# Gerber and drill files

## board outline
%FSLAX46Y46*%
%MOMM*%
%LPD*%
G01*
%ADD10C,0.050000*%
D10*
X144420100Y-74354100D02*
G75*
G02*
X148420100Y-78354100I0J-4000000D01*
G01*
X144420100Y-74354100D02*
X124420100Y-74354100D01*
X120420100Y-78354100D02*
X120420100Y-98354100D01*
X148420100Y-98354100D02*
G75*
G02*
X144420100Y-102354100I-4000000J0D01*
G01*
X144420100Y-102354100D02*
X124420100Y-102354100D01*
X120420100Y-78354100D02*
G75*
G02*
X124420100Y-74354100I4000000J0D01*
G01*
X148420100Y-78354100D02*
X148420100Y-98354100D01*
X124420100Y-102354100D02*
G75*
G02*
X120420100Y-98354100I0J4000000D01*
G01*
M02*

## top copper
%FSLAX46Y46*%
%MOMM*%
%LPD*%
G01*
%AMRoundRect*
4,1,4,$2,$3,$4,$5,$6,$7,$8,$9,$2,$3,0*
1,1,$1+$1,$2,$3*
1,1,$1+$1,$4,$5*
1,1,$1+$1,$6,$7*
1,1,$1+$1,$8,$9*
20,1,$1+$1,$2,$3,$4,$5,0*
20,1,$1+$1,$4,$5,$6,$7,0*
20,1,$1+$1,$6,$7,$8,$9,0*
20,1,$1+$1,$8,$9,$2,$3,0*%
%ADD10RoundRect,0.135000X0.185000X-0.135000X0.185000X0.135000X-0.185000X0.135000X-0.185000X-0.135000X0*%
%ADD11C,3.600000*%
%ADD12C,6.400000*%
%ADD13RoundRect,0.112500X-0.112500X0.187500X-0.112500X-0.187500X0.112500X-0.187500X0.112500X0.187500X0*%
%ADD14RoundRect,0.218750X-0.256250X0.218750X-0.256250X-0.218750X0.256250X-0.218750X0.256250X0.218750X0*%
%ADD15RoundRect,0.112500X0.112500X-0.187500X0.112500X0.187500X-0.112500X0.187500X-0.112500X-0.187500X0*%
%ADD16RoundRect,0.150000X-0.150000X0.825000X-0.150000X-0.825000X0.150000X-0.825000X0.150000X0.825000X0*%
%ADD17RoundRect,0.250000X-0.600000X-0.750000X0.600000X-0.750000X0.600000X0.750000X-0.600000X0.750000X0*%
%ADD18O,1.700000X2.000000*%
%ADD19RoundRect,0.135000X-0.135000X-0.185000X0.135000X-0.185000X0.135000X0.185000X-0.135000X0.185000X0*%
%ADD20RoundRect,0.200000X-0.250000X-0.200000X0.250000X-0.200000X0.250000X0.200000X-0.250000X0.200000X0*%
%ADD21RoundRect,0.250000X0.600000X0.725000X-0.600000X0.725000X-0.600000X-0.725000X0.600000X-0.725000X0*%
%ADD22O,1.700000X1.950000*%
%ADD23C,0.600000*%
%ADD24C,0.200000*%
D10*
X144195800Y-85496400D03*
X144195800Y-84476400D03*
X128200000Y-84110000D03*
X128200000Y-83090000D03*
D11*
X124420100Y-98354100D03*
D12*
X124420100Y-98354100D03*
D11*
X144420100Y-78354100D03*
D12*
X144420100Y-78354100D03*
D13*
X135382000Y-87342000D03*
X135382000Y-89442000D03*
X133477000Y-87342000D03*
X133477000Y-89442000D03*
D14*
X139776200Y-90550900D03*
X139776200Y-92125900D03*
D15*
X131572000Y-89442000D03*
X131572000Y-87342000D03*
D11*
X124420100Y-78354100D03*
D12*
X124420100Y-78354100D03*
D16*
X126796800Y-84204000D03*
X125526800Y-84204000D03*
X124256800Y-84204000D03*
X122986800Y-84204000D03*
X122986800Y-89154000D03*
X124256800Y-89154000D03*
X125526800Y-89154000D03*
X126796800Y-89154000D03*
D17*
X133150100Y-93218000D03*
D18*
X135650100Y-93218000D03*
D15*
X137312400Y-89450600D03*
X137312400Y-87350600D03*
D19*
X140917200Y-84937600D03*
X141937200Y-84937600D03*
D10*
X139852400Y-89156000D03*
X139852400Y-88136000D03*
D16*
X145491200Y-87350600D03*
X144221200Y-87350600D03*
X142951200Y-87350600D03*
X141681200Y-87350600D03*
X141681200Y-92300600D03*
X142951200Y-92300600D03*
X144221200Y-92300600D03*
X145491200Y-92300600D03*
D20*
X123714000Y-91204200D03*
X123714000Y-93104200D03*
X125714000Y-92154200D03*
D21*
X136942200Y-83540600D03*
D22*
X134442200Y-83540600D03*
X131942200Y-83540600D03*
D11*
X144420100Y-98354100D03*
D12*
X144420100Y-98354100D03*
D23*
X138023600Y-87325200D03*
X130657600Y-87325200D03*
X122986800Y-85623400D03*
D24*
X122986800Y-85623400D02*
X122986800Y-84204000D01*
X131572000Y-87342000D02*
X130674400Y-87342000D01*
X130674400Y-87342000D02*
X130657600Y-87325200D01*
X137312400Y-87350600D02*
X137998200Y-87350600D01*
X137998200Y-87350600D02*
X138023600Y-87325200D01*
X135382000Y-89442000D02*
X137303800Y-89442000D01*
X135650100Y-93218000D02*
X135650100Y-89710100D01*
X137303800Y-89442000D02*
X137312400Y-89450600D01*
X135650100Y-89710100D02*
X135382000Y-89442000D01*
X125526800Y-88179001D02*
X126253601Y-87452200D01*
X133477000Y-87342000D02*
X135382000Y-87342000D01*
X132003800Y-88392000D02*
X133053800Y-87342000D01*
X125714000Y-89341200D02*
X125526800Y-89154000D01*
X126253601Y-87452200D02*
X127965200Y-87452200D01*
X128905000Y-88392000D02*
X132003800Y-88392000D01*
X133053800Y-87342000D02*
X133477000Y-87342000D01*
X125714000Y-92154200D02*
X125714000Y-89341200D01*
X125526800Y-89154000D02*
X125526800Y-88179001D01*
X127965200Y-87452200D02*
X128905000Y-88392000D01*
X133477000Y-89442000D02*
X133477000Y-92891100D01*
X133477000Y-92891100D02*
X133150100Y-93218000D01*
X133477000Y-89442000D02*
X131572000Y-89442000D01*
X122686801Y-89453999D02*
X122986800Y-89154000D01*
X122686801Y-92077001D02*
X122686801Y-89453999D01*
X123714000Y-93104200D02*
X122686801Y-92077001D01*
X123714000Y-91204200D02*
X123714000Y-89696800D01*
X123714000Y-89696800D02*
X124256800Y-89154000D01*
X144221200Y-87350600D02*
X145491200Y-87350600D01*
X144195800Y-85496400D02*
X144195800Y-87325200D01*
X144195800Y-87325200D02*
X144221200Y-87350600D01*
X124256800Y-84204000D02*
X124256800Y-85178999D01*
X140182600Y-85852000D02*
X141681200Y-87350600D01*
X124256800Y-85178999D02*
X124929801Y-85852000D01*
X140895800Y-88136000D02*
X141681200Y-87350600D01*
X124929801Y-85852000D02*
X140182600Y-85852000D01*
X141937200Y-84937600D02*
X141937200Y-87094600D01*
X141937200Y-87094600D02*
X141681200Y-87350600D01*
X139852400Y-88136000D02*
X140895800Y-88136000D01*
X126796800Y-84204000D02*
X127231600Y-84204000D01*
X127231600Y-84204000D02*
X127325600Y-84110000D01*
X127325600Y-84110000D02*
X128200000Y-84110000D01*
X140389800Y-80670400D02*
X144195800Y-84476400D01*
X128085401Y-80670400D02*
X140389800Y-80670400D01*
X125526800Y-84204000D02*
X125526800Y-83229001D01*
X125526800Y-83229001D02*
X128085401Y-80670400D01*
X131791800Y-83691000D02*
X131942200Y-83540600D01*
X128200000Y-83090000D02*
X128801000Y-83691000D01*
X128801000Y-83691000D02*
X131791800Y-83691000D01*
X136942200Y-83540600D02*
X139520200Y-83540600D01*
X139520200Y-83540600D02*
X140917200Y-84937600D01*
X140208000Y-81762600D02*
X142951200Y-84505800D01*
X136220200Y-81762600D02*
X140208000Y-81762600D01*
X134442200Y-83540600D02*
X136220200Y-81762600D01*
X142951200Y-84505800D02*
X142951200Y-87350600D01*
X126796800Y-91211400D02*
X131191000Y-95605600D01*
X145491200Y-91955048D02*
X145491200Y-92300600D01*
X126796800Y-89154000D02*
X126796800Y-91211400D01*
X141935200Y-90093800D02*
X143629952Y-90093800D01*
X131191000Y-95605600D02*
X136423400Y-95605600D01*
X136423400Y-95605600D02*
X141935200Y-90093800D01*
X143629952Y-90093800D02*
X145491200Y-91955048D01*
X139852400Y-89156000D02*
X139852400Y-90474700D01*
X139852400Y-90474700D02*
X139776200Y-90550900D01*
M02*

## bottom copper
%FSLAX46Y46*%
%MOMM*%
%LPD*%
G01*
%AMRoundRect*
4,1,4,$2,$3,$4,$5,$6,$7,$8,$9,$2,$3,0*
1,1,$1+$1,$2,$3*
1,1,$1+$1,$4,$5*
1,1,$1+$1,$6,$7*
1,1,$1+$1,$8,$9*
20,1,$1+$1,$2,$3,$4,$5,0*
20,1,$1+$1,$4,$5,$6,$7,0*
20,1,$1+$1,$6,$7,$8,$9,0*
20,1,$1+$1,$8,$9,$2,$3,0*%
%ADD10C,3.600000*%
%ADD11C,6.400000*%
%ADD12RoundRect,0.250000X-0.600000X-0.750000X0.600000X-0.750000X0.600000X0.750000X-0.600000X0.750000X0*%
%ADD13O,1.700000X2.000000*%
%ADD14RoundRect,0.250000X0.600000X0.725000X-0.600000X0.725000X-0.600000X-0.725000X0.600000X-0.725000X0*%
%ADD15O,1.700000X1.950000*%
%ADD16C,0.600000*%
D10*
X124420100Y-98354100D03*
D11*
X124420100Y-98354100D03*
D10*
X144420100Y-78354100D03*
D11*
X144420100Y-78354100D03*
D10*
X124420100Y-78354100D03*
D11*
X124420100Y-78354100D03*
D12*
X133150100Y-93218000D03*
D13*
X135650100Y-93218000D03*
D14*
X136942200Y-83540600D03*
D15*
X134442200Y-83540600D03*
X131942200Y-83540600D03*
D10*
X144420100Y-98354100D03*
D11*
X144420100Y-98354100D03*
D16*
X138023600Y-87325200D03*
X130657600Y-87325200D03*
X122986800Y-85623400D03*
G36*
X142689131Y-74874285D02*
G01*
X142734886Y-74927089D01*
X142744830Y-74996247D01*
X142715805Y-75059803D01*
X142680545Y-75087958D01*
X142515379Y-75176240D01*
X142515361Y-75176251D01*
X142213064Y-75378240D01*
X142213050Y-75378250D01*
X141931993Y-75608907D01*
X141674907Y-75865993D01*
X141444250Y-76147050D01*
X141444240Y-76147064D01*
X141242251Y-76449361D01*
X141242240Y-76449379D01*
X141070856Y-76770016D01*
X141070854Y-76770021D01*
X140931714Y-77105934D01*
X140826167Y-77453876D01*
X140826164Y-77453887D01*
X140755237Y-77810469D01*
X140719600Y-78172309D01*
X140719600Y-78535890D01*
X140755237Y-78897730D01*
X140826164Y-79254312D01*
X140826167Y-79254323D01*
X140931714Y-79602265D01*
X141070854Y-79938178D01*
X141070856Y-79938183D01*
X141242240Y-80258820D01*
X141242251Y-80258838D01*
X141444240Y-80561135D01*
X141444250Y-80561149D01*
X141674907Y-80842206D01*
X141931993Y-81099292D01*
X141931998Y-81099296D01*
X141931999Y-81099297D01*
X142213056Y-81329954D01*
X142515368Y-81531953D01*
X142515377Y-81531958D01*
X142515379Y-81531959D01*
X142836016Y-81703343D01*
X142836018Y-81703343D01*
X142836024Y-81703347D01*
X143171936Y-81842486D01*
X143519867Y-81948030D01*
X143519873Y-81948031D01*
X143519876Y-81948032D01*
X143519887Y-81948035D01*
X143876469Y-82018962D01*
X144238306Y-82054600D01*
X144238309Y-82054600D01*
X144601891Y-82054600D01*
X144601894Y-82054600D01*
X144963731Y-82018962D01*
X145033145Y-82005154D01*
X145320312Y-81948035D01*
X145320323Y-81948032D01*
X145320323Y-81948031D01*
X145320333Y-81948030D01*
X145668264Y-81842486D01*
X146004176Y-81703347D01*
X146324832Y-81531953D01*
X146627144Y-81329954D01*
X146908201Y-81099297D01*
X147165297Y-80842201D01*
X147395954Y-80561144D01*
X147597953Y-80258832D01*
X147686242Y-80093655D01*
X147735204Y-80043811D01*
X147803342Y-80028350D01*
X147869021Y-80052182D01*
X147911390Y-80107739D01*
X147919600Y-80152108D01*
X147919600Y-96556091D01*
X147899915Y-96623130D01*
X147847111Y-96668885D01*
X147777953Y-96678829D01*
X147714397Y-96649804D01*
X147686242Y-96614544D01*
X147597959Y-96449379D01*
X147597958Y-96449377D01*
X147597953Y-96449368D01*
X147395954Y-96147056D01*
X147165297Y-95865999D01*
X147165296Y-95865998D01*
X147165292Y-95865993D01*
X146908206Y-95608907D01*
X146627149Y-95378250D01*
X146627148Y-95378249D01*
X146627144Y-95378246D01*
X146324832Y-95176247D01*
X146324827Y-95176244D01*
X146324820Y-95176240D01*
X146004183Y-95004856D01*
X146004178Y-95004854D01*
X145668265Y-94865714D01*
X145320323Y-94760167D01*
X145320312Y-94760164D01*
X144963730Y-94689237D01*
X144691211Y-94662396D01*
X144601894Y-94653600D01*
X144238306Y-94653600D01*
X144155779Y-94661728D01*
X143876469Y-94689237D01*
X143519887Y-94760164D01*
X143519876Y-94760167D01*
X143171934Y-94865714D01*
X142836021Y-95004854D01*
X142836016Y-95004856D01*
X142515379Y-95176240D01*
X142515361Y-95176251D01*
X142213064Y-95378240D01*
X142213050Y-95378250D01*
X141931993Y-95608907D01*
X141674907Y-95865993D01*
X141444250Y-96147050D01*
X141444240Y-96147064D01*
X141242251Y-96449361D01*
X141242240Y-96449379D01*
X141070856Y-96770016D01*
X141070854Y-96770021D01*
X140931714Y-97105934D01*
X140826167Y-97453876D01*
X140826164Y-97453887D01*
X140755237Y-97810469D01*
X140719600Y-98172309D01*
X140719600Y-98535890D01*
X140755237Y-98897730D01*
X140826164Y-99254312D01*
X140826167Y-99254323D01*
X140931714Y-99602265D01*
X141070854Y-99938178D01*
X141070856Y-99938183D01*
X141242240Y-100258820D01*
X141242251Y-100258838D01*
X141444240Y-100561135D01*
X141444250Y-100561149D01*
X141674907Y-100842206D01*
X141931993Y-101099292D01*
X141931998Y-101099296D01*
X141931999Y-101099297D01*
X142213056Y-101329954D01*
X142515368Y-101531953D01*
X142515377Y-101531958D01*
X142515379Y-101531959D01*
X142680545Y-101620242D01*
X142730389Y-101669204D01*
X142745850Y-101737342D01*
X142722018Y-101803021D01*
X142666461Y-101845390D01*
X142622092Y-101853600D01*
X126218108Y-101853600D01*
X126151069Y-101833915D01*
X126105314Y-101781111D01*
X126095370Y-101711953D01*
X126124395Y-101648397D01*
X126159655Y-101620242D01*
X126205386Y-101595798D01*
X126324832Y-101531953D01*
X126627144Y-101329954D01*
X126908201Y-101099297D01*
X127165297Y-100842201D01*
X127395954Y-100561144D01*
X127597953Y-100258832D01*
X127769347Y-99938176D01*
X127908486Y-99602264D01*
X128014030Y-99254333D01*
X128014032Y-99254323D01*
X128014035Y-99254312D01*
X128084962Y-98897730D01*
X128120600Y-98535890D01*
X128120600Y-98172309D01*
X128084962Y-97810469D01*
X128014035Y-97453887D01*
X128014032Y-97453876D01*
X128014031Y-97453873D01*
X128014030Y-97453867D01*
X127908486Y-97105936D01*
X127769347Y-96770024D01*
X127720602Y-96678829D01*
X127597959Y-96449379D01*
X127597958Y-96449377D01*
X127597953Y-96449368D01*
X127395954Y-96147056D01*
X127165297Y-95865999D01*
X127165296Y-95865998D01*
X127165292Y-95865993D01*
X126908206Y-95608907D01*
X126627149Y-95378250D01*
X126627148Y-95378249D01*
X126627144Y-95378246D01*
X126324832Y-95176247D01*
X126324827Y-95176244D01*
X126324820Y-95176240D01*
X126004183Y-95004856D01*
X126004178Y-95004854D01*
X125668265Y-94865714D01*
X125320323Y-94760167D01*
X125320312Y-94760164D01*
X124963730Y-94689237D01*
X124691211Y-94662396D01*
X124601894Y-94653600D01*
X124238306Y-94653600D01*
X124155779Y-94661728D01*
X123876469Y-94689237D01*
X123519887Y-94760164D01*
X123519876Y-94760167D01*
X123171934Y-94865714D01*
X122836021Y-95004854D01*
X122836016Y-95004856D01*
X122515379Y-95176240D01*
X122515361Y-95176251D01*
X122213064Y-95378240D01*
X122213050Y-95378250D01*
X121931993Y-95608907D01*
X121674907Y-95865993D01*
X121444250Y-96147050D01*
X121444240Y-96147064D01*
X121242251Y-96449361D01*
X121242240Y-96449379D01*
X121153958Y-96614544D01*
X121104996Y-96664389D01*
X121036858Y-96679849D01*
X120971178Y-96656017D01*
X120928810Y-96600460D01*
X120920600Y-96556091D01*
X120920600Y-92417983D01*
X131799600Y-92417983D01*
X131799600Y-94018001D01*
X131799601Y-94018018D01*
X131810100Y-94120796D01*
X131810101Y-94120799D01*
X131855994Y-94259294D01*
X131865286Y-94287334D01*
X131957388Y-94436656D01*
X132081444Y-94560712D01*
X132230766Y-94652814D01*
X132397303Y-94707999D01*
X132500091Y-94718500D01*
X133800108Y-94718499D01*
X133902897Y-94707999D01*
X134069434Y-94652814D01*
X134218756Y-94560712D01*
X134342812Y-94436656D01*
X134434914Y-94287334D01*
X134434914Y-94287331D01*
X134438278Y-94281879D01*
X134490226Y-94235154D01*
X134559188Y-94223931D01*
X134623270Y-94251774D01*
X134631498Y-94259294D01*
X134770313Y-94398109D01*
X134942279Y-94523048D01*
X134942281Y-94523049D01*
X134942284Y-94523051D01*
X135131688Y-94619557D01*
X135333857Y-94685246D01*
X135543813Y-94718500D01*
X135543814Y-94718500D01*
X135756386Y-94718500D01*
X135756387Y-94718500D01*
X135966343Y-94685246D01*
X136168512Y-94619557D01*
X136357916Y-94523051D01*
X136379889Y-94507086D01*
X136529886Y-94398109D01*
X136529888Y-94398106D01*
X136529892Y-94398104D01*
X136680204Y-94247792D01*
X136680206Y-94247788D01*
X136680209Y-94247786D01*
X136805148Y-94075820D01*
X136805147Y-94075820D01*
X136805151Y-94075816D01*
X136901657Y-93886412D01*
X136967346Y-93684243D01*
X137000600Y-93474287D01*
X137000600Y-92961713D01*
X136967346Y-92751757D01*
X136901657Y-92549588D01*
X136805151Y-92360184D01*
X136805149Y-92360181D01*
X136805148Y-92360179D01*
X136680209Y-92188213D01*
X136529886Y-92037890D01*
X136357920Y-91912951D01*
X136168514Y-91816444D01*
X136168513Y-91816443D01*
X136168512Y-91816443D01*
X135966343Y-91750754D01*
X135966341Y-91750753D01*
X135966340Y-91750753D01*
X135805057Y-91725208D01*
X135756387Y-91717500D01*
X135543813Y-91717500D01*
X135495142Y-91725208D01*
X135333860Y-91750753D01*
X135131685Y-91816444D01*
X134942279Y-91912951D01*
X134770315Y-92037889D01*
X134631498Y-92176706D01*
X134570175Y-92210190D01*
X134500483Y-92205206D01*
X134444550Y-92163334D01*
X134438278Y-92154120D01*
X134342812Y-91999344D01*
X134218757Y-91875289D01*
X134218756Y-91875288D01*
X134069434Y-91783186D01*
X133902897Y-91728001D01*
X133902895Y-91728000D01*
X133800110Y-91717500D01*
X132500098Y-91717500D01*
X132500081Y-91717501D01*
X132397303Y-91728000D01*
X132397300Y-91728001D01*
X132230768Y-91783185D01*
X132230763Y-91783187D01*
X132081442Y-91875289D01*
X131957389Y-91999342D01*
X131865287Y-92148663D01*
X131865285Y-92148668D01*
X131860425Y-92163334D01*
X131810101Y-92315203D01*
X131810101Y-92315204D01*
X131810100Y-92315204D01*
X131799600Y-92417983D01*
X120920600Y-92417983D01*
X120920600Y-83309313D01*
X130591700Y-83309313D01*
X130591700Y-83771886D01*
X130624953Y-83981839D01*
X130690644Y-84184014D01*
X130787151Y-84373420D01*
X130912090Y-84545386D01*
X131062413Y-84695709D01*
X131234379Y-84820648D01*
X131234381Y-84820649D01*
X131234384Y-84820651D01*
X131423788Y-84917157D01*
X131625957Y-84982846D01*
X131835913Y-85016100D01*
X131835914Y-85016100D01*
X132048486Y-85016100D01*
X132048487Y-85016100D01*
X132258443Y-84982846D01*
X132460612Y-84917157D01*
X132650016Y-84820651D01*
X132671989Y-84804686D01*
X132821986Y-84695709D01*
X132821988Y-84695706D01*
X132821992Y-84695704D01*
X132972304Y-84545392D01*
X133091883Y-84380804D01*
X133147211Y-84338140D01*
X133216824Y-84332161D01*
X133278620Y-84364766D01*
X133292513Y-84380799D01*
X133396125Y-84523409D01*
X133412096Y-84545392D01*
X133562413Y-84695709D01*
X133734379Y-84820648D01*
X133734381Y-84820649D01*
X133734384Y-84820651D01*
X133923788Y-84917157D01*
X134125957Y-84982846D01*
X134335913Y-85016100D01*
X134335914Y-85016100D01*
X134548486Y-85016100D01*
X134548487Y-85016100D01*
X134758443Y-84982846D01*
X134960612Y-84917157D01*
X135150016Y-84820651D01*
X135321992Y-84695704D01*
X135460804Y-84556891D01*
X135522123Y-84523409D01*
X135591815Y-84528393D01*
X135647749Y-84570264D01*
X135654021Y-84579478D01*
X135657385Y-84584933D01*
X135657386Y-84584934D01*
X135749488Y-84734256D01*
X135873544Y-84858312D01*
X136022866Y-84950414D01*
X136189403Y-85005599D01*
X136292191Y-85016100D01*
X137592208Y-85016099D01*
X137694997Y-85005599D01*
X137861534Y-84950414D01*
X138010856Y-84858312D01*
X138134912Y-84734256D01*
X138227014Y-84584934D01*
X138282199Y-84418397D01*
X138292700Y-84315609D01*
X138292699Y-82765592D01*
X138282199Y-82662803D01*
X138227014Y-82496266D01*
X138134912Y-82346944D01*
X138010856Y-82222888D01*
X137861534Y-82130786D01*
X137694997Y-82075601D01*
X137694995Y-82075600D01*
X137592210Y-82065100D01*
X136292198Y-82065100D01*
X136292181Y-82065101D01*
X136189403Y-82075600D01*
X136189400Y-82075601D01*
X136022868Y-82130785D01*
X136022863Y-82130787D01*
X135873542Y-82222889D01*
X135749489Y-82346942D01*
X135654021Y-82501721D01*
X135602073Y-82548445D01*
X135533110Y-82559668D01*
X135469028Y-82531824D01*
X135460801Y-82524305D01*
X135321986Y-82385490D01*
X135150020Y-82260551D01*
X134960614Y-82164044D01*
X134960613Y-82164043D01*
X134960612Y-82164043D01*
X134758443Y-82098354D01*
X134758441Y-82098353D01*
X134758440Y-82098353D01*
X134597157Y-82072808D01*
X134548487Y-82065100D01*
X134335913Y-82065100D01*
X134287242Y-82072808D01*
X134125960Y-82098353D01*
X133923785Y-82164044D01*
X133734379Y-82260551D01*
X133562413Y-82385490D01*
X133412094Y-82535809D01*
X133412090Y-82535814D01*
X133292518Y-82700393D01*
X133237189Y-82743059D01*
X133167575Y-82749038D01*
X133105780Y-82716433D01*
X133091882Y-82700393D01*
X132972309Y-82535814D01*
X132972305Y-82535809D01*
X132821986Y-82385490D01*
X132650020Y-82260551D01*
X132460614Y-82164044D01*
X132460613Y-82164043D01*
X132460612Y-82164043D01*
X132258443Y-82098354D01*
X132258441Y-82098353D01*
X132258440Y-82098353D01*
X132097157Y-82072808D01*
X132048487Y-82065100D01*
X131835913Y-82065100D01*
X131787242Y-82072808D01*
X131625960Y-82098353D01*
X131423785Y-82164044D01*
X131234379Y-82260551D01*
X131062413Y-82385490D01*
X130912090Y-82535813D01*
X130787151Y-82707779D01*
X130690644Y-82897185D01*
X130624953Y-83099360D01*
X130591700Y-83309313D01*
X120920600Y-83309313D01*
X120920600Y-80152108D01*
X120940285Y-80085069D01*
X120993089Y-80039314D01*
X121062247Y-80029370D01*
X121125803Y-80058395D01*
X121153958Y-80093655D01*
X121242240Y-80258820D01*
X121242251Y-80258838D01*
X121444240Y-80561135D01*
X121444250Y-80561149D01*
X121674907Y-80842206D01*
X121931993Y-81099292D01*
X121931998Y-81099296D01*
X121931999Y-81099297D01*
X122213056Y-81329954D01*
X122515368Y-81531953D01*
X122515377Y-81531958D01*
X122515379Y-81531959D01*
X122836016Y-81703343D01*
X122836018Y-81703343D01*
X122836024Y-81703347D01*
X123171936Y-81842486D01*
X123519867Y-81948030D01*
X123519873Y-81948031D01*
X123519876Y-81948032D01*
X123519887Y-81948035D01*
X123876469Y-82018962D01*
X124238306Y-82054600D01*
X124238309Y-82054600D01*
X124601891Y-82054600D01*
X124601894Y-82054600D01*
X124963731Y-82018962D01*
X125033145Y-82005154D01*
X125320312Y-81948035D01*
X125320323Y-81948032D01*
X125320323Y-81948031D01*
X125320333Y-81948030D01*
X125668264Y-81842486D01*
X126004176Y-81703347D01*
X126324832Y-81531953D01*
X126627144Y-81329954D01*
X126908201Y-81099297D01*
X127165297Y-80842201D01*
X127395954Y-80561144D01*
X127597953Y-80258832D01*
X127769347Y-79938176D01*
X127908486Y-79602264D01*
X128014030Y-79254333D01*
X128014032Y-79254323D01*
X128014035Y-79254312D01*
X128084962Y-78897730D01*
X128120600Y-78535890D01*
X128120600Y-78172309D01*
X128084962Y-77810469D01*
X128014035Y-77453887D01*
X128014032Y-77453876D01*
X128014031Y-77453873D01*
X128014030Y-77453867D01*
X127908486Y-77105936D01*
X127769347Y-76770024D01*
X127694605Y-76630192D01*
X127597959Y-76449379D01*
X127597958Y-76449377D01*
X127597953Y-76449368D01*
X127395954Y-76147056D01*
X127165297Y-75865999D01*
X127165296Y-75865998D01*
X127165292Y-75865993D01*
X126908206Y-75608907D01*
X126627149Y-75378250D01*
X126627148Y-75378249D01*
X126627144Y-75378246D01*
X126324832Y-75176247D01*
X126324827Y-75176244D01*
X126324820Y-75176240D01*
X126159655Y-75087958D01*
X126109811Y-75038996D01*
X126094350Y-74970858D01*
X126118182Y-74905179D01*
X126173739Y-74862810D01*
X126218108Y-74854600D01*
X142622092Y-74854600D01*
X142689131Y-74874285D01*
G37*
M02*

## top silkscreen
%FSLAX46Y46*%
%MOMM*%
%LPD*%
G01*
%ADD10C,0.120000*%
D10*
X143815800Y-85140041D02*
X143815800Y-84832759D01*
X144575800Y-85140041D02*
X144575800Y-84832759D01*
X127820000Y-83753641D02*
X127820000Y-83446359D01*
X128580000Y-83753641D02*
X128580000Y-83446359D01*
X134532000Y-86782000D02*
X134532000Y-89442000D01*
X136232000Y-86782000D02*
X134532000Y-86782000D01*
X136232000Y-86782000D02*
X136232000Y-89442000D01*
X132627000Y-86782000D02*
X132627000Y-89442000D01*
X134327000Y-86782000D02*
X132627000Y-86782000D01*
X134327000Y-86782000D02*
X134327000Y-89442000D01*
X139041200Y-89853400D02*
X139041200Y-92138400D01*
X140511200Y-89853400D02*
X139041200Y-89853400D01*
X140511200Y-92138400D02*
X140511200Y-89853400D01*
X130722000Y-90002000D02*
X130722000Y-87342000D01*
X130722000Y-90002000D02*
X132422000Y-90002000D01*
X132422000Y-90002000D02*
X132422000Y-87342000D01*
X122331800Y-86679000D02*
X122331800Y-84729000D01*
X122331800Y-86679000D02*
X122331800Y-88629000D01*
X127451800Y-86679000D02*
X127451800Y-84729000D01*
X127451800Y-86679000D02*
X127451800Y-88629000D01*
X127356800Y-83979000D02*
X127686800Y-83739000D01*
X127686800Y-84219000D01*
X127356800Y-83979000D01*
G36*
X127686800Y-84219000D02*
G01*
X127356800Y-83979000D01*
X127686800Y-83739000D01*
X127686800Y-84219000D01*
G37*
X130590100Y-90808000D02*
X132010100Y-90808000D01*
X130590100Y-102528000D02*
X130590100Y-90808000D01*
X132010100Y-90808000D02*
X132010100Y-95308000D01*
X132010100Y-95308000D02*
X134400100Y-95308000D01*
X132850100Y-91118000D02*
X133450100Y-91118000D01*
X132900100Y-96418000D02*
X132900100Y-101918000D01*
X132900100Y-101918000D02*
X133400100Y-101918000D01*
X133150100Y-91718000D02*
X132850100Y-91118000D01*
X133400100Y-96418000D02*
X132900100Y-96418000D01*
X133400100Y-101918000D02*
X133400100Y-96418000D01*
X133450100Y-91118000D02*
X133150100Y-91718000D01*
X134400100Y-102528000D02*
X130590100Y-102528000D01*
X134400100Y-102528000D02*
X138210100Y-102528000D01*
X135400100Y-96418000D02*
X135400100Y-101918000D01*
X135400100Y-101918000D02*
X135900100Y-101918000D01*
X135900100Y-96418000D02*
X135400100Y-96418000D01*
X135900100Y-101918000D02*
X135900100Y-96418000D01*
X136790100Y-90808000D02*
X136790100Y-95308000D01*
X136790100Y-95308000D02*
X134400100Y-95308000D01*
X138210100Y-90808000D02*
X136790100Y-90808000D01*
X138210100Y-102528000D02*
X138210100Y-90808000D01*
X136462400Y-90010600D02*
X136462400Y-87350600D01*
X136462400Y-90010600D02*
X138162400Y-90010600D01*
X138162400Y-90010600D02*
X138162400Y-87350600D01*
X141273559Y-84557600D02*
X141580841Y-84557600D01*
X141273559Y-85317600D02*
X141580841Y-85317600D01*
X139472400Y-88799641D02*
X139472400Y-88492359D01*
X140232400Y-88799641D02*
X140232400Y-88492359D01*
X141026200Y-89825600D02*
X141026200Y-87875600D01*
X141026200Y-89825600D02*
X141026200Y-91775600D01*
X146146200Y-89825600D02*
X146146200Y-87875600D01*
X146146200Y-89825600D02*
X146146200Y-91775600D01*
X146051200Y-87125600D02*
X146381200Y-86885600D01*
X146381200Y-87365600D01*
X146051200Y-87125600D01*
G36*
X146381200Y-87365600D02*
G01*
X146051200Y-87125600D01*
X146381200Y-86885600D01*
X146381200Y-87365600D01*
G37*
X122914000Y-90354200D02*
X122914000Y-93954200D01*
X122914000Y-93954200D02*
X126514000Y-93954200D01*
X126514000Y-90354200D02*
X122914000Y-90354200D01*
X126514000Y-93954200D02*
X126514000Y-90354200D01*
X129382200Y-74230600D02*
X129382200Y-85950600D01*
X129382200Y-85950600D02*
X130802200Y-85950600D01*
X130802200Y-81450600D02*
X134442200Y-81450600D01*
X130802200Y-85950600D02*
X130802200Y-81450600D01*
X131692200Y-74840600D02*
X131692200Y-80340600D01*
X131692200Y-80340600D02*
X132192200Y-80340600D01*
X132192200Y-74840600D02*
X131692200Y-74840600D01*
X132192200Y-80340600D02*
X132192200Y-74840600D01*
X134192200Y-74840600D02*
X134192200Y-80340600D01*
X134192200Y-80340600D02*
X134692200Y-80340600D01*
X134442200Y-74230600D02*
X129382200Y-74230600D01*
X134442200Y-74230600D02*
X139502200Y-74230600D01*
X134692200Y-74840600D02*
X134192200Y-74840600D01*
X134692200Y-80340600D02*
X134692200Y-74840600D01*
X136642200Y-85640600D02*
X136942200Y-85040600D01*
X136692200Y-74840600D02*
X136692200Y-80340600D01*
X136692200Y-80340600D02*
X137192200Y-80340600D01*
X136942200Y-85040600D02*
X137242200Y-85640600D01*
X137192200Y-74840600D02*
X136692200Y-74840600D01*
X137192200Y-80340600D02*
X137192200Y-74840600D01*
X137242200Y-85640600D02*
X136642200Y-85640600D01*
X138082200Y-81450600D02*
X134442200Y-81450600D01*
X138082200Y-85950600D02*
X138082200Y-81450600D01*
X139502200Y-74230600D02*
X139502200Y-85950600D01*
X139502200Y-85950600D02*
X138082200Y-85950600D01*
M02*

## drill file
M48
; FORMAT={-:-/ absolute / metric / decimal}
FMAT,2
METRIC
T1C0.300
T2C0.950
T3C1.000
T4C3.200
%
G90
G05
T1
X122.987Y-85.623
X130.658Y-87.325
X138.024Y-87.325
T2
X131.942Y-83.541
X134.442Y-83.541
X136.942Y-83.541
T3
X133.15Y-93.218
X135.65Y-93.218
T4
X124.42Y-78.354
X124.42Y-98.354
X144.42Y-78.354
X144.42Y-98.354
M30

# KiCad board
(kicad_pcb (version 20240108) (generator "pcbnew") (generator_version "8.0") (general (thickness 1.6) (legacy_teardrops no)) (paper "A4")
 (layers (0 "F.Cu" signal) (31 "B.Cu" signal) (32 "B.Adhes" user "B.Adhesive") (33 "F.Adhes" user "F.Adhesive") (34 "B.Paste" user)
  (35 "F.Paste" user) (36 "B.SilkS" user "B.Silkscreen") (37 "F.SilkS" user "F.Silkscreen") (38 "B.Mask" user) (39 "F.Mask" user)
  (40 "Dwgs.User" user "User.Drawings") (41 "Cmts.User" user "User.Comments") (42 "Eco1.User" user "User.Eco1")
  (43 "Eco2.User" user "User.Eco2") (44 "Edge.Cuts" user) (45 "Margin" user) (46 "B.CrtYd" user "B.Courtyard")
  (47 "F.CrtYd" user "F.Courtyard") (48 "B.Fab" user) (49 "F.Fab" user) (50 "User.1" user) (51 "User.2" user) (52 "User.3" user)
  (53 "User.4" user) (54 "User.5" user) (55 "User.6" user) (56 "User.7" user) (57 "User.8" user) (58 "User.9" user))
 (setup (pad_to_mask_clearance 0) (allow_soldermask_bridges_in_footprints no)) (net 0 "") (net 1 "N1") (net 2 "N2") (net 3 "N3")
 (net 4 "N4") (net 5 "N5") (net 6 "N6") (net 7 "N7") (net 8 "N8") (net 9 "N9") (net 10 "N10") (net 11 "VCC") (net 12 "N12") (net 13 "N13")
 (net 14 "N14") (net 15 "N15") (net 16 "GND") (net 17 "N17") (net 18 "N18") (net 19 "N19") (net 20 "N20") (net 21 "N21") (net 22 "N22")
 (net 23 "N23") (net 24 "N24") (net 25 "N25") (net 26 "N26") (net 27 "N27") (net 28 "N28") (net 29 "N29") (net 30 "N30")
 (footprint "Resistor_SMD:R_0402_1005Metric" (layer "F.Cu") (at 144.1958 84.9864 90)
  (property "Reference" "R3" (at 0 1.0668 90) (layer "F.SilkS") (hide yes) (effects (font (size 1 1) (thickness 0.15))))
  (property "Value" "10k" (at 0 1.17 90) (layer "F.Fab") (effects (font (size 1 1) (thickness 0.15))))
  (fp_line (start -0.153641 -0.38) (end 0.153641 -0.38) (stroke (width 0.12) (type solid)) (layer "F.SilkS"))
  (fp_line (start -0.153641 0.38) (end 0.153641 0.38) (stroke (width 0.12) (type solid)) (layer "F.SilkS"))
  (pad "1" smd roundrect (at -0.51 0 90) (size 0.54 0.64) (layers "F.Cu" "F.Paste" "F.Mask") (roundrect_rratio 0.25) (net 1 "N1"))
  (pad "2" smd roundrect (at 0.51 0 90) (size 0.54 0.64) (layers "F.Cu" "F.Paste" "F.Mask") (roundrect_rratio 0.25) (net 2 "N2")))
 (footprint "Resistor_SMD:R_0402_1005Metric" (layer "F.Cu") (at 128.2 83.6 90)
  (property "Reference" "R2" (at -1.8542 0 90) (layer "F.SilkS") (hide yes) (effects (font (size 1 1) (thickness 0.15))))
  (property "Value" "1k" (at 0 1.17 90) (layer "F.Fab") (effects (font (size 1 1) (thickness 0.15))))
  (fp_line (start -0.153641 -0.38) (end 0.153641 -0.38) (stroke (width 0.12) (type solid)) (layer "F.SilkS"))
  (fp_line (start -0.153641 0.38) (end 0.153641 0.38) (stroke (width 0.12) (type solid)) (layer "F.SilkS"))
  (pad "1" smd roundrect (at -0.51 0 90) (size 0.54 0.64) (layers "F.Cu" "F.Paste" "F.Mask") (roundrect_rratio 0.25) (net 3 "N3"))
  (pad "2" smd roundrect (at 0.51 0 90) (size 0.54 0.64) (layers "F.Cu" "F.Paste" "F.Mask") (roundrect_rratio 0.25) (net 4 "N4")))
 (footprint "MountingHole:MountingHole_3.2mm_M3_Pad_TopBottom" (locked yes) (layer "F.Cu") (at 124.4201 98.3541)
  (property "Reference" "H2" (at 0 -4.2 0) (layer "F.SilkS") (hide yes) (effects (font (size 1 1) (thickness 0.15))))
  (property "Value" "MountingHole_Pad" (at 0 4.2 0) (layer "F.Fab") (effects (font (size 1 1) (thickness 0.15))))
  (pad "1" thru_hole circle (at 0 0) (size 3.6 3.6) (drill 3.2) (layers "*.Cu" "*.Mask") (remove_unused_layers no) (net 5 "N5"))
  (pad "1" connect circle (at 0 0) (size 6.4 6.4) (layers "F.Cu" "F.Mask") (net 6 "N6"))
  (pad "1" connect circle (at 0 0) (size 6.4 6.4) (layers "B.Cu" "B.Mask") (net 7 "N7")))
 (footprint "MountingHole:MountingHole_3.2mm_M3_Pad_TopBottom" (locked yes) (layer "F.Cu") (at 144.4201 78.3541)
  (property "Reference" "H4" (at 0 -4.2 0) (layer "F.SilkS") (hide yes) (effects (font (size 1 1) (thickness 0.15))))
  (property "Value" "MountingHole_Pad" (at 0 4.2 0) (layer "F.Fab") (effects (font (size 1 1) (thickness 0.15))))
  (pad "1" thru_hole circle (at 0 0) (size 3.6 3.6) (drill 3.2) (layers "*.Cu" "*.Mask") (remove_unused_layers no) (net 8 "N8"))
  (pad "1" connect circle (at 0 0) (size 6.4 6.4) (layers "F.Cu" "F.Mask") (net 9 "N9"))
  (pad "1" connect circle (at 0 0) (size 6.4 6.4) (layers "B.Cu" "B.Mask") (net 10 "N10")))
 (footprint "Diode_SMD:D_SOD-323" (layer "F.Cu") (at 135.382 88.392 -90)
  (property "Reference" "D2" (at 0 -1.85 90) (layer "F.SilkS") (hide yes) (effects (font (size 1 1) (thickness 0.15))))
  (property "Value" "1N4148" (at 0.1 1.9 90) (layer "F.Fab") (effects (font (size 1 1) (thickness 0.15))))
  (fp_line (start -1.61 0.85) (end 1.05 0.85) (stroke (width 0.12) (type solid)) (layer "F.SilkS"))
  (fp_line (start -1.61 -0.85) (end -1.61 0.85) (stroke (width 0.12) (type solid)) (layer "F.SilkS"))
  (fp_line (start -1.61 -0.85) (end 1.05 -0.85) (stroke (width 0.12) (type solid)) (layer "F.SilkS"))
  (pad "1" smd roundrect (at -1.05 0 270) (size 0.6 0.45) (layers "F.Cu" "F.Paste" "F.Mask") (roundrect_rratio 0.25) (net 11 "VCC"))
  (pad "2" smd roundrect (at 1.05 0 270) (size 0.6 0.45) (layers "F.Cu" "F.Paste" "F.Mask") (roundrect_rratio 0.25) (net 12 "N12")))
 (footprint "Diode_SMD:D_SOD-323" (layer "F.Cu") (at 133.477 88.392 -90)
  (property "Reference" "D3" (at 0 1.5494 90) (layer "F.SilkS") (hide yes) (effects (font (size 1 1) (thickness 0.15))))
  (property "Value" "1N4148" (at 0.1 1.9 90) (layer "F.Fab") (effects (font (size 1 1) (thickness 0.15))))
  (fp_line (start -1.61 0.85) (end 1.05 0.85) (stroke (width 0.12) (type solid)) (layer "F.SilkS"))
  (fp_line (start -1.61 -0.85) (end -1.61 0.85) (stroke (width 0.12) (type solid)) (layer "F.SilkS"))
  (fp_line (start -1.61 -0.85) (end 1.05 -0.85) (stroke (width 0.12) (type solid)) (layer "F.SilkS"))
  (pad "1" smd roundrect (at -1.05 0 270) (size 0.6 0.45) (layers "F.Cu" "F.Paste" "F.Mask") (roundrect_rratio 0.25) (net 11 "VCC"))
  (pad "2" smd roundrect (at 1.05 0 270) (size 0.6 0.45) (layers "F.Cu" "F.Paste" "F.Mask") (roundrect_rratio 0.25) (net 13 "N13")))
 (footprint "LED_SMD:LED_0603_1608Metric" (layer "F.Cu") (at 139.7762 91.3384 -90)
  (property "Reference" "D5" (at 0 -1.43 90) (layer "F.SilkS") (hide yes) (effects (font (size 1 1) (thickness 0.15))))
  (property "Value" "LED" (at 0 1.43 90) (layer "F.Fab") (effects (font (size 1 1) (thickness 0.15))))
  (fp_line (start -1.485 0.735) (end 0.8 0.735) (stroke (width 0.12) (type solid)) (layer "F.SilkS"))
  (fp_line (start -1.485 -0.735) (end -1.485 0.735) (stroke (width 0.12) (type solid)) (layer "F.SilkS"))
  (fp_line (start 0.8 -0.735) (end -1.485 -0.735) (stroke (width 0.12) (type solid)) (layer "F.SilkS"))
  (pad "1" smd roundrect (at -0.7875 0 270) (size 0.875 0.95) (layers "F.Cu" "F.Paste" "F.Mask") (roundrect_rratio 0.25) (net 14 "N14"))
  (pad "2" smd roundrect (at 0.7875 0 270) (size 0.875 0.95) (layers "F.Cu" "F.Paste" "F.Mask") (roundrect_rratio 0.25) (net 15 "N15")))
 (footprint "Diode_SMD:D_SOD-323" (layer "F.Cu") (at 131.572 88.392 90)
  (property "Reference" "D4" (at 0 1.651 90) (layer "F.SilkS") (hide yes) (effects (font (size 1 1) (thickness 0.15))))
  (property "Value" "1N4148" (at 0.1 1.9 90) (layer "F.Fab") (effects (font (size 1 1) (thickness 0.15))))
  (fp_line (start -1.61 -0.85) (end 1.05 -0.85) (stroke (width 0.12) (type solid)) (layer "F.SilkS"))
  (fp_line (start -1.61 -0.85) (end -1.61 0.85) (stroke (width 0.12) (type solid)) (layer "F.SilkS"))
  (fp_line (start -1.61 0.85) (end 1.05 0.85) (stroke (width 0.12) (type solid)) (layer "F.SilkS"))
  (pad "1" smd roundrect (at -1.05 0 90) (size 0.6 0.45) (layers "F.Cu" "F.Paste" "F.Mask") (roundrect_rratio 0.25) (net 13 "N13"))
  (pad "2" smd roundrect (at 1.05 0 90) (size 0.6 0.45) (layers "F.Cu" "F.Paste" "F.Mask") (roundrect_rratio 0.25) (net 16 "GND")))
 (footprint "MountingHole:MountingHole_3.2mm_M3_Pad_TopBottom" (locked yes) (layer "F.Cu") (at 124.4201 78.3541)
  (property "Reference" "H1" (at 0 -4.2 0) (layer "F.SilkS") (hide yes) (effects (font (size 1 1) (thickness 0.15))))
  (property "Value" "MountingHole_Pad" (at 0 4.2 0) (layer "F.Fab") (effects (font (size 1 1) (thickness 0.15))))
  (pad "1" thru_hole circle (at 0 0) (size 3.6 3.6) (drill 3.2) (layers "*.Cu" "*.Mask") (remove_unused_layers no) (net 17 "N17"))
  (pad "1" connect circle (at 0 0) (size 6.4 6.4) (layers "F.Cu" "F.Mask") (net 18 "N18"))
  (pad "1" connect circle (at 0 0) (size 6.4 6.4) (layers "B.Cu" "B.Mask") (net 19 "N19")))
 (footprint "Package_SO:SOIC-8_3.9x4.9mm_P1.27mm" (layer "F.Cu") (at 124.8918 86.679 -90)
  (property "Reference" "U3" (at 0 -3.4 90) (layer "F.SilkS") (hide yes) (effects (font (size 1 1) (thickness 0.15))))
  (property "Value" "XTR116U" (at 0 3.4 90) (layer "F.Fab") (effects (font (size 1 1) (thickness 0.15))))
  (fp_line (start 0 2.56) (end -1.95 2.56) (stroke (width 0.12) (type solid)) (layer "F.SilkS"))
  (fp_line (start 0 2.56) (end 1.95 2.56) (stroke (width 0.12) (type solid)) (layer "F.SilkS"))
  (fp_line (start 0 -2.56) (end -1.95 -2.56) (stroke (width 0.12) (type solid)) (layer "F.SilkS"))
  (fp_line (start 0 -2.56) (end 1.95 -2.56) (stroke (width 0.12) (type solid)) (layer "F.SilkS"))
  (fp_poly
   (pts (xy -2.7 -2.465) (xy -2.94 -2.795) (xy -2.46 -2.795) (xy -2.7 -2.465)) (stroke (width 0.12) (type solid)) (fill solid)
   (layer "F.SilkS"))
  (pad "1" smd roundrect (at -2.475 -1.905 270) (size 1.95 0.6) (layers "F.Cu" "F.Paste" "F.Mask") (roundrect_rratio 0.25) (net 3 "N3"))
  (pad "2" smd roundrect (at -2.475 -0.635 270) (size 1.95 0.6) (layers "F.Cu" "F.Paste" "F.Mask") (roundrect_rratio 0.25) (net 2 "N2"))
  (pad "3" smd roundrect (at -2.475 0.635 270) (size 1.95 0.6) (layers "F.Cu" "F.Paste" "F.Mask") (roundrect_rratio 0.25) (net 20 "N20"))
  (pad "4" smd roundrect (at -2.475 1.905 270) (size 1.95 0.6) (layers "F.Cu" "F.Paste" "F.Mask") (roundrect_rratio 0.25) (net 16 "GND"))
  (pad "5" smd roundrect (at 2.475 1.905 270) (size 1.95 0.6) (layers "F.Cu" "F.Paste" "F.Mask") (roundrect_rratio 0.25) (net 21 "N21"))
  (pad "6" smd roundrect (at 2.475 0.635 270) (size 1.95 0.6) (layers "F.Cu" "F.Paste" "F.Mask") (roundrect_rratio 0.25) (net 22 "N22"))
  (pad "7" smd roundrect (at 2.475 -0.635 270) (size 1.95 0.6) (layers "F.Cu" "F.Paste" "F.Mask") (roundrect_rratio 0.25) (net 11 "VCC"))
  (pad "8" smd roundrect (at 2.475 -1.905 270) (size 1.95 0.6) (layers "F.Cu" "F.Paste" "F.Mask") (roundrect_rratio 0.25) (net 15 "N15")))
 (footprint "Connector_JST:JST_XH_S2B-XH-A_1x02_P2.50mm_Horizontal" (layer "F.Cu") (at 133.1501 93.218)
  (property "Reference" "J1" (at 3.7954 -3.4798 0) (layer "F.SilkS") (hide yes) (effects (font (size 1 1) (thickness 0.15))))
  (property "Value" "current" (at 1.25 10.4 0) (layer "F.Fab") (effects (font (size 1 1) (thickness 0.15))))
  (fp_line (start -2.56 -2.41) (end -1.14 -2.41) (stroke (width 0.12) (type solid)) (layer "F.SilkS"))
  (fp_line (start -2.56 9.31) (end -2.56 -2.41) (stroke (width 0.12) (type solid)) (layer "F.SilkS"))
  (fp_line (start -1.14 -2.41) (end -1.14 2.09) (stroke (width 0.12) (type solid)) (layer "F.SilkS"))
  (fp_line (start -1.14 2.09) (end 1.25 2.09) (stroke (width 0.12) (type solid)) (layer "F.SilkS"))
  (fp_line (start -0.3 -2.1) (end 0.3 -2.1) (stroke (width 0.12) (type solid)) (layer "F.SilkS"))
  (fp_line (start -0.25 3.2) (end -0.25 8.7) (stroke (width 0.12) (type solid)) (layer "F.SilkS"))
  (fp_line (start -0.25 8.7) (end 0.25 8.7) (stroke (width 0.12) (type solid)) (layer "F.SilkS"))
  (fp_line (start 0 -1.5) (end -0.3 -2.1) (stroke (width 0.12) (type solid)) (layer "F.SilkS"))
  (fp_line (start 0.25 3.2) (end -0.25 3.2) (stroke (width 0.12) (type solid)) (layer "F.SilkS"))
  (fp_line (start 0.25 8.7) (end 0.25 3.2) (stroke (width 0.12) (type solid)) (layer "F.SilkS"))
  (fp_line (start 0.3 -2.1) (end 0 -1.5) (stroke (width 0.12) (type solid)) (layer "F.SilkS"))
  (fp_line (start 1.25 9.31) (end -2.56 9.31) (stroke (width 0.12) (type solid)) (layer "F.SilkS"))
  (fp_line (start 1.25 9.31) (end 5.06 9.31) (stroke (width 0.12) (type solid)) (layer "F.SilkS"))
  (fp_line (start 2.25 3.2) (end 2.25 8.7) (stroke (width 0.12) (type solid)) (layer "F.SilkS"))
  (fp_line (start 2.25 8.7) (end 2.75 8.7) (stroke (width 0.12) (type solid)) (layer "F.SilkS"))
  (fp_line (start 2.75 3.2) (end 2.25 3.2) (stroke (width 0.12) (type solid)) (layer "F.SilkS"))
  (fp_line (start 2.75 8.7) (end 2.75 3.2) (stroke (width 0.12) (type solid)) (layer "F.SilkS"))
  (fp_line (start 3.64 -2.41) (end 3.64 2.09) (stroke (width 0.12) (type solid)) (layer "F.SilkS"))
  (fp_line (start 3.64 2.09) (end 1.25 2.09) (stroke (width 0.12) (type solid)) (layer "F.SilkS"))
  (fp_line (start 5.06 -2.41) (end 3.64 -2.41) (stroke (width 0.12) (type solid)) (layer "F.SilkS"))
  (fp_line (start 5.06 9.31) (end 5.06 -2.41) (stroke (width 0.12) (type solid)) (layer "F.SilkS"))
  (pad "1" thru_hole roundrect (at 0 0) (size 1.7 2) (drill 1) (layers "*.Cu" "*.Mask") (remove_unused_layers no)
   (roundrect_rratio 0.147059) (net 13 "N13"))
  (pad "2" thru_hole oval (at 2.5 0) (size 1.7 2) (drill 1) (layers "*.Cu" "*.Mask") (remove_unused_layers no) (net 12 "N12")))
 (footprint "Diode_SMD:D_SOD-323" (layer "F.Cu") (at 137.3124 88.4006 90)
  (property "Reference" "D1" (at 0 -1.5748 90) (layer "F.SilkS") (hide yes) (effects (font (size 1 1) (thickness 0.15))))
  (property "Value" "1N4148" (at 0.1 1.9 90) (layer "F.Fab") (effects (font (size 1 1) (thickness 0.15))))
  (fp_line (start -1.61 -0.85) (end 1.05 -0.85) (stroke (width 0.12) (type solid)) (layer "F.SilkS"))
  (fp_line (start -1.61 -0.85) (end -1.61 0.85) (stroke (width 0.12) (type solid)) (layer "F.SilkS"))
  (fp_line (start -1.61 0.85) (end 1.05 0.85) (stroke (width 0.12) (type solid)) (layer "F.SilkS"))
  (pad "1" smd roundrect (at -1.05 0 90) (size 0.6 0.45) (layers "F.Cu" "F.Paste" "F.Mask") (roundrect_rratio 0.25) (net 12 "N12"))
  (pad "2" smd roundrect (at 1.05 0 90) (size 0.6 0.45) (layers "F.Cu" "F.Paste" "F.Mask") (roundrect_rratio 0.25) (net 16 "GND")))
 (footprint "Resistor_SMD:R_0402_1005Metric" (layer "F.Cu") (at 141.4272 84.9376)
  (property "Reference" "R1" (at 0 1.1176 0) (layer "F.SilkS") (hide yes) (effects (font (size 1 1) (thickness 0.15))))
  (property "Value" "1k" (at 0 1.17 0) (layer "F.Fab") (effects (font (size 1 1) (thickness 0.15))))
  (fp_line (start -0.153641 -0.38) (end 0.153641 -0.38) (stroke (width 0.12) (type solid)) (layer "F.SilkS"))
  (fp_line (start -0.153641 0.38) (end 0.153641 0.38) (stroke (width 0.12) (type solid)) (layer "F.SilkS"))
  (pad "1" smd roundrect (at -0.51 0) (size 0.54 0.64) (layers "F.Cu" "F.Paste" "F.Mask") (roundrect_rratio 0.25) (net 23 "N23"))
  (pad "2" smd roundrect (at 0.51 0) (size 0.54 0.64) (layers "F.Cu" "F.Paste" "F.Mask") (roundrect_rratio 0.25) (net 20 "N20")))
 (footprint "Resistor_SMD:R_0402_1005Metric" (layer "F.Cu") (at 139.8524 88.646 90)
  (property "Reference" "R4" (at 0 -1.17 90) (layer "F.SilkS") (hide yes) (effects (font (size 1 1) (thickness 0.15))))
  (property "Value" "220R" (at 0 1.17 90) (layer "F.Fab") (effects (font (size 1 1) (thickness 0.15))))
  (fp_line (start -0.153641 -0.38) (end 0.153641 -0.38) (stroke (width 0.12) (type solid)) (layer "F.SilkS"))
  (fp_line (start -0.153641 0.38) (end 0.153641 0.38) (stroke (width 0.12) (type solid)) (layer "F.SilkS"))
  (pad "1" smd roundrect (at -0.51 0 90) (size 0.54 0.64) (layers "F.Cu" "F.Paste" "F.Mask") (roundrect_rratio 0.25) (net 14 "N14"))
  (pad "2" smd roundrect (at 0.51 0 90) (size 0.54 0.64) (layers "F.Cu" "F.Paste" "F.Mask") (roundrect_rratio 0.25) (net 20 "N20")))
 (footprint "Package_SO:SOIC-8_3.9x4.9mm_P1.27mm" (layer "F.Cu") (at 143.5862 89.8256 -90)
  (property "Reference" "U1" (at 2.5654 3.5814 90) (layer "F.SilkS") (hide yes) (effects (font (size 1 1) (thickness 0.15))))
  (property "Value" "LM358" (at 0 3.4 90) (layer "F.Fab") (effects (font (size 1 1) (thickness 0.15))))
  (fp_line (start 0 2.56) (end -1.95 2.56) (stroke (width 0.12) (type solid)) (layer "F.SilkS"))
  (fp_line (start 0 2.56) (end 1.95 2.56) (stroke (width 0.12) (type solid)) (layer "F.SilkS"))
  (fp_line (start 0 -2.56) (end -1.95 -2.56) (stroke (width 0.12) (type solid)) (layer "F.SilkS"))
  (fp_line (start 0 -2.56) (end 1.95 -2.56) (stroke (width 0.12) (type solid)) (layer "F.SilkS"))
  (fp_poly
   (pts (xy -2.7 -2.465) (xy -2.94 -2.795) (xy -2.46 -2.795) (xy -2.7 -2.465)) (stroke (width 0.12) (type solid)) (fill solid)
   (layer "F.SilkS"))
  (pad "1" smd roundrect (at -2.475 -1.905 270) (size 1.95 0.6) (layers "F.Cu" "F.Paste" "F.Mask") (roundrect_rratio 0.25) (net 1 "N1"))
  (pad "2" smd roundrect (at -2.475 -0.635 270) (size 1.95 0.6) (layers "F.Cu" "F.Paste" "F.Mask") (roundrect_rratio 0.25) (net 1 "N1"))
  (pad "3" smd roundrect (at -2.475 0.635 270) (size 1.95 0.6) (layers "F.Cu" "F.Paste" "F.Mask") (roundrect_rratio 0.25) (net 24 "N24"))
  (pad "4" smd roundrect (at -2.475 1.905 270) (size 1.95 0.6) (layers "F.Cu" "F.Paste" "F.Mask") (roundrect_rratio 0.25) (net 20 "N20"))
  (pad "5" smd roundrect (at 2.475 1.905 270) (size 1.95 0.6) (layers "F.Cu" "F.Paste" "F.Mask") (roundrect_rratio 0.25) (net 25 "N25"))
  (pad "6" smd roundrect (at 2.475 0.635 270) (size 1.95 0.6) (layers "F.Cu" "F.Paste" "F.Mask") (roundrect_rratio 0.25) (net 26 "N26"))
  (pad "7" smd roundrect (at 2.475 -0.635 270) (size 1.95 0.6) (layers "F.Cu" "F.Paste" "F.Mask") (roundrect_rratio 0.25) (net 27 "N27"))
  (pad "8" smd roundrect (at 2.475 -1.905 270) (size 1.95 0.6) (layers "F.Cu" "F.Paste" "F.Mask") (roundrect_rratio 0.25) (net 15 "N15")))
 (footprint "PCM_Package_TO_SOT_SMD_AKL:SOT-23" (layer "F.Cu") (at 124.714 92.1542)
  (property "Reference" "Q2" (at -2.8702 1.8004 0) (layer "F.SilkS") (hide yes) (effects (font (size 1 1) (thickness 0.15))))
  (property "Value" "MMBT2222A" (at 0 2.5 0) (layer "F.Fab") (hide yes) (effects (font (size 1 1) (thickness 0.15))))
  (fp_line (start -1.8 -1.8) (end -1.8 1.8) (stroke (width 0.12) (type solid)) (layer "F.SilkS"))
  (fp_line (start -1.8 1.8) (end 1.8 1.8) (stroke (width 0.12) (type solid)) (layer "F.SilkS"))
  (fp_line (start 1.8 -1.8) (end -1.8 -1.8) (stroke (width 0.12) (type solid)) (layer "F.SilkS"))
  (fp_line (start 1.8 1.8) (end 1.8 -1.8) (stroke (width 0.12) (type solid)) (layer "F.SilkS"))
  (pad "1" smd roundrect (at -1 -0.95) (size 0.9 0.8) (layers "F.Cu" "F.Paste" "F.Mask") (roundrect_rratio 0.25) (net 22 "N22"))
  (pad "2" smd roundrect (at -1 0.95) (size 0.9 0.8) (layers "F.Cu" "F.Paste" "F.Mask") (roundrect_rratio 0.25) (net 21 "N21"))
  (pad "3" smd roundrect (at 1 0) (size 0.9 0.8) (layers "F.Cu" "F.Paste" "F.Mask") (roundrect_rratio 0.25) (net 11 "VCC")))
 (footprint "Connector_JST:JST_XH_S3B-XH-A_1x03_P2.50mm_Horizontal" (layer "F.Cu") (at 136.9422 83.5406 180)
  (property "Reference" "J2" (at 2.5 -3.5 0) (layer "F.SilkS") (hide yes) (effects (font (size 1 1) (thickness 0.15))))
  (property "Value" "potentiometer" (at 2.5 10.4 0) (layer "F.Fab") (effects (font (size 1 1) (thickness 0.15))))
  (fp_line (start 7.56 9.31) (end 7.56 -2.41) (stroke (width 0.12) (type solid)) (layer "F.SilkS"))
  (fp_line (start 7.56 -2.41) (end 6.14 -2.41) (stroke (width 0.12) (type solid)) (layer "F.SilkS"))
  (fp_line (start 6.14 2.09) (end 2.5 2.09) (stroke (width 0.12) (type solid)) (layer "F.SilkS"))
  (fp_line (start 6.14 -2.41) (end 6.14 2.09) (stroke (width 0.12) (type solid)) (layer "F.SilkS"))
  (fp_line (start 5.25 8.7) (end 5.25 3.2) (stroke (width 0.12) (type solid)) (layer "F.SilkS"))
  (fp_line (start 5.25 3.2) (end 4.75 3.2) (stroke (width 0.12) (type solid)) (layer "F.SilkS"))
  (fp_line (start 4.75 8.7) (end 5.25 8.7) (stroke (width 0.12) (type solid)) (layer "F.SilkS"))
  (fp_line (start 4.75 3.2) (end 4.75 8.7) (stroke (width 0.12) (type solid)) (layer "F.SilkS"))
  (fp_line (start 2.75 8.7) (end 2.75 3.2) (stroke (width 0.12) (type solid)) (layer "F.SilkS"))
  (fp_line (start 2.75 3.2) (end 2.25 3.2) (stroke (width 0.12) (type solid)) (layer "F.SilkS"))
  (fp_line (start 2.5 9.31) (end 7.56 9.31) (stroke (width 0.12) (type solid)) (layer "F.SilkS"))
  (fp_line (start 2.5 9.31) (end -2.56 9.31) (stroke (width 0.12) (type solid)) (layer "F.SilkS"))
  (fp_line (start 2.25 8.7) (end 2.75 8.7) (stroke (width 0.12) (type solid)) (layer "F.SilkS"))
  (fp_line (start 2.25 3.2) (end 2.25 8.7) (stroke (width 0.12) (type solid)) (layer "F.SilkS"))
  (fp_line (start 0.3 -2.1) (end 0 -1.5) (stroke (width 0.12) (type solid)) (layer "F.SilkS"))
  (fp_line (start 0.25 8.7) (end 0.25 3.2) (stroke (width 0.12) (type solid)) (layer "F.SilkS"))
  (fp_line (start 0.25 3.2) (end -0.25 3.2) (stroke (width 0.12) (type solid)) (layer "F.SilkS"))
  (fp_line (start 0 -1.5) (end -0.3 -2.1) (stroke (width 0.12) (type solid)) (layer "F.SilkS"))
  (fp_line (start -0.25 8.7) (end 0.25 8.7) (stroke (width 0.12) (type solid)) (layer "F.SilkS"))
  (fp_line (start -0.25 3.2) (end -0.25 8.7) (stroke (width 0.12) (type solid)) (layer "F.SilkS"))
  (fp_line (start -0.3 -2.1) (end 0.3 -2.1) (stroke (width 0.12) (type solid)) (layer "F.SilkS"))
  (fp_line (start -1.14 2.09) (end 2.5 2.09) (stroke (width 0.12) (type solid)) (layer "F.SilkS"))
  (fp_line (start -1.14 -2.41) (end -1.14 2.09) (stroke (width 0.12) (type solid)) (layer "F.SilkS"))
  (fp_line (start -2.56 9.31) (end -2.56 -2.41) (stroke (width 0.12) (type solid)) (layer "F.SilkS"))
  (fp_line (start -2.56 -2.41) (end -1.14 -2.41) (stroke (width 0.12) (type solid)) (layer "F.SilkS"))
  (pad "1" thru_hole roundrect (at 0 0 180) (size 1.7 1.95) (drill 0.95) (layers "*.Cu" "*.Mask") (remove_unused_layers no)
   (roundrect_rratio 0.147059) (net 23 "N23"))
  (pad "2" thru_hole oval (at 2.5 0 180) (size 1.7 1.95) (drill 0.95) (layers "*.Cu" "*.Mask") (remove_unused_layers no) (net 24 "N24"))
  (pad "3" thru_hole oval (at 5 0 180) (size 1.7 1.95) (drill 0.95) (layers "*.Cu" "*.Mask") (remove_unused_layers no) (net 4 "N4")))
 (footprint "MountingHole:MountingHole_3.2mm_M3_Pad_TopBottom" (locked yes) (layer "F.Cu") (at 144.4201 98.3541)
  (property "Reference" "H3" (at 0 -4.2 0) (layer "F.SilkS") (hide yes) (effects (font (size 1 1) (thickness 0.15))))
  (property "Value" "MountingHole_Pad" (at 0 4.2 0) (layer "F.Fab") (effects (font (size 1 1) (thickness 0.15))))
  (pad "1" thru_hole circle (at 0 0) (size 3.6 3.6) (drill 3.2) (layers "*.Cu" "*.Mask") (remove_unused_layers no) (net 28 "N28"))
  (pad "1" connect circle (at 0 0) (size 6.4 6.4) (layers "F.Cu" "F.Mask") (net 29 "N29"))
  (pad "1" connect circle (at 0 0) (size 6.4 6.4) (layers "B.Cu" "B.Mask") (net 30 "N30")))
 (gr_arc (start 144.4201 74.3541) (mid 147.248527 75.525673) (end 148.4201 78.3541) (stroke (width 0.05) (type default)) (layer "Edge.Cuts"))
 (gr_line (start 144.4201 74.3541) (end 124.4201 74.3541) (stroke (width 0.05) (type default)) (layer "Edge.Cuts"))
 (gr_line (start 120.4201 78.3541) (end 120.4201 98.3541) (stroke (width 0.05) (type default)) (layer "Edge.Cuts"))
 (gr_arc (start 148.4201 98.3541) (mid 147.248527 101.182527) (end 144.4201 102.3541) (stroke (width 0.05) (type default))
  (layer "Edge.Cuts"))
 (gr_line (start 144.4201 102.3541) (end 124.4201 102.3541) (stroke (width 0.05) (type default)) (layer "Edge.Cuts"))
 (gr_arc (start 120.4201 78.3541) (mid 121.591673 75.525673) (end 124.4201 74.3541) (stroke (width 0.05) (type default)) (layer "Edge.Cuts"))
 (gr_line (start 148.4201 78.3541) (end 148.4201 98.3541) (stroke (width 0.05) (type default)) (layer "Edge.Cuts"))
 (gr_arc (start 124.4201 102.3541) (mid 121.591673 101.182527) (end 120.4201 98.3541) (stroke (width 0.05) (type default))
  (layer "Edge.Cuts"))
 (segment (start 122.9868 85.6234) (end 122.9868 84.204) (width 0.2) (layer "F.Cu") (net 16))
 (segment (start 131.572 87.342) (end 130.6744 87.342) (width 0.2) (layer "F.Cu") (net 16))
 (segment (start 130.6744 87.342) (end 130.6576 87.3252) (width 0.2) (layer "F.Cu") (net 16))
 (segment (start 137.3124 87.3506) (end 137.9982 87.3506) (width 0.2) (layer "F.Cu") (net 16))
 (segment (start 137.9982 87.3506) (end 138.0236 87.3252) (width 0.2) (layer "F.Cu") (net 16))
 (via (at 138.0236 87.3252) (size 0.6) (drill 0.3) (layers "F.Cu" "B.Cu") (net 16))
 (via (at 130.6576 87.3252) (size 0.6) (drill 0.3) (layers "F.Cu" "B.Cu") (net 16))
 (via (at 122.9868 85.6234) (size 0.6) (drill 0.3) (layers "F.Cu" "B.Cu") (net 16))
 (segment (start 135.382 89.442) (end 137.3038 89.442) (width 0.2) (layer "F.Cu") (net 12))
 (segment (start 135.6501 93.218) (end 135.6501 89.7101) (width 0.2) (layer "F.Cu") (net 12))
 (segment (start 137.3038 89.442) (end 137.3124 89.4506) (width 0.2) (layer "F.Cu") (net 12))
 (segment (start 135.6501 89.7101) (end 135.382 89.442) (width 0.2) (layer "F.Cu") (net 12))
 (segment (start 125.5268 88.179001) (end 126.253601 87.4522) (width 0.2) (layer "F.Cu") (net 11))
 (segment (start 133.477 87.342) (end 135.382 87.342) (width 0.2) (layer "F.Cu") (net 11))
 (segment (start 132.0038 88.392) (end 133.0538 87.342) (width 0.2) (layer "F.Cu") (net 11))
 (segment (start 125.714 89.3412) (end 125.5268 89.154) (width 0.2) (layer "F.Cu") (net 11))
 (segment (start 126.253601 87.4522) (end 127.9652 87.4522) (width 0.2) (layer "F.Cu") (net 11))
 (segment (start 128.905 88.392) (end 132.0038 88.392) (width 0.2) (layer "F.Cu") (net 11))
 (segment (start 133.0538 87.342) (end 133.477 87.342) (width 0.2) (layer "F.Cu") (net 11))
 (segment (start 125.714 92.1542) (end 125.714 89.3412) (width 0.2) (layer "F.Cu") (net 11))
 (segment (start 125.5268 89.154) (end 125.5268 88.179001) (width 0.2) (layer "F.Cu") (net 11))
 (segment (start 127.9652 87.4522) (end 128.905 88.392) (width 0.2) (layer "F.Cu") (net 11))
 (segment (start 133.477 89.442) (end 133.477 92.8911) (width 0.2) (layer "F.Cu") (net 13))
 (segment (start 133.477 92.8911) (end 133.1501 93.218) (width 0.2) (layer "F.Cu") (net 13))
 (segment (start 133.477 89.442) (end 131.572 89.442) (width 0.2) (layer "F.Cu") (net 13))
 (segment (start 122.686801 89.453999) (end 122.9868 89.154) (width 0.2) (layer "F.Cu") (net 21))
 (segment (start 122.686801 92.077001) (end 122.686801 89.453999) (width 0.2) (layer "F.Cu") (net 21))
 (segment (start 123.714 93.1042) (end 122.686801 92.077001) (width 0.2) (layer "F.Cu") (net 21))
 (segment (start 123.714 91.2042) (end 123.714 89.6968) (width 0.2) (layer "F.Cu") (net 22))
 (segment (start 123.714 89.6968) (end 124.2568 89.154) (width 0.2) (layer "F.Cu") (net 22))
 (segment (start 144.2212 87.3506) (end 145.4912 87.3506) (width 0.2) (layer "F.Cu") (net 1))
 (segment (start 144.1958 85.4964) (end 144.1958 87.3252) (width 0.2) (layer "F.Cu") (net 1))
 (segment (start 144.1958 87.3252) (end 144.2212 87.3506) (width 0.2) (layer "F.Cu") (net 1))
 (segment (start 124.2568 84.204) (end 124.2568 85.178999) (width 0.2) (layer "F.Cu") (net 20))
 (segment (start 140.1826 85.852) (end 141.6812 87.3506) (width 0.2) (layer "F.Cu") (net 20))
 (segment (start 124.2568 85.178999) (end 124.929801 85.852) (width 0.2) (layer "F.Cu") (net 20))
 (segment (start 140.8958 88.136) (end 141.6812 87.3506) (width 0.2) (layer "F.Cu") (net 20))
 (segment (start 124.929801 85.852) (end 140.1826 85.852) (width 0.2) (layer "F.Cu") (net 20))
 (segment (start 141.9372 84.9376) (end 141.9372 87.0946) (width 0.2) (layer "F.Cu") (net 20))
 (segment (start 141.9372 87.0946) (end 141.6812 87.3506) (width 0.2) (layer "F.Cu") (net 20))
 (segment (start 139.8524 88.136) (end 140.8958 88.136) (width 0.2) (layer "F.Cu") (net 20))
 (segment (start 126.7968 84.204) (end 127.2316 84.204) (width 0.2) (layer "F.Cu") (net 3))
 (segment (start 127.2316 84.204) (end 127.3256 84.11) (width 0.2) (layer "F.Cu") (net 3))
 (segment (start 127.3256 84.11) (end 128.2 84.11) (width 0.2) (layer "F.Cu") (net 3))
 (segment (start 140.3898 80.6704) (end 144.1958 84.4764) (width 0.2) (layer "F.Cu") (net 2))
 (segment (start 128.085401 80.6704) (end 140.3898 80.6704) (width 0.2) (layer "F.Cu") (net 2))
 (segment (start 125.5268 84.204) (end 125.5268 83.229001) (width 0.2) (layer "F.Cu") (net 2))
 (segment (start 125.5268 83.229001) (end 128.085401 80.6704) (width 0.2) (layer "F.Cu") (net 2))
 (segment (start 131.7918 83.691) (end 131.9422 83.5406) (width 0.2) (layer "F.Cu") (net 4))
 (segment (start 128.2 83.09) (end 128.801 83.691) (width 0.2) (layer "F.Cu") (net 4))
 (segment (start 128.801 83.691) (end 131.7918 83.691) (width 0.2) (layer "F.Cu") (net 4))
 (segment (start 136.9422 83.5406) (end 139.5202 83.5406) (width 0.2) (layer "F.Cu") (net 23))
 (segment (start 139.5202 83.5406) (end 140.9172 84.9376) (width 0.2) (layer "F.Cu") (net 23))
 (segment (start 140.208 81.7626) (end 142.9512 84.5058) (width 0.2) (layer "F.Cu") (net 24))
 (segment (start 136.2202 81.7626) (end 140.208 81.7626) (width 0.2) (layer "F.Cu") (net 24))
 (segment (start 134.4422 83.5406) (end 136.2202 81.7626) (width 0.2) (layer "F.Cu") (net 24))
 (segment (start 142.9512 84.5058) (end 142.9512 87.3506) (width 0.2) (layer "F.Cu") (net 24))
 (segment (start 126.7968 91.2114) (end 131.191 95.6056) (width 0.2) (layer "F.Cu") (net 15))
 (segment (start 145.4912 91.955048) (end 145.4912 92.3006) (width 0.2) (layer "F.Cu") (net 15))
 (segment (start 126.7968 89.154) (end 126.7968 91.2114) (width 0.2) (layer "F.Cu") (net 15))
 (segment (start 141.9352 90.0938) (end 143.629952 90.0938) (width 0.2) (layer "F.Cu") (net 15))
 (segment (start 131.191 95.6056) (end 136.4234 95.6056) (width 0.2) (layer "F.Cu") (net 15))
 (segment (start 136.4234 95.6056) (end 141.9352 90.0938) (width 0.2) (layer "F.Cu") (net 15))
 (segment (start 143.629952 90.0938) (end 145.4912 91.955048) (width 0.2) (layer "F.Cu") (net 15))
 (segment (start 139.8524 89.156) (end 139.8524 90.4747) (width 0.2) (layer "F.Cu") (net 14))
 (segment (start 139.8524 90.4747) (end 139.7762 90.5509) (width 0.2) (layer "F.Cu") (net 14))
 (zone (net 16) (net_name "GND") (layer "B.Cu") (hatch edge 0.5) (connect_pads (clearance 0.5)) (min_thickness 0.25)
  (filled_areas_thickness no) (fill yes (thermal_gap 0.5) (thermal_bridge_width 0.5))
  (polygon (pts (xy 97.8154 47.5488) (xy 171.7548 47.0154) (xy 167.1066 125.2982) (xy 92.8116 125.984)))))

